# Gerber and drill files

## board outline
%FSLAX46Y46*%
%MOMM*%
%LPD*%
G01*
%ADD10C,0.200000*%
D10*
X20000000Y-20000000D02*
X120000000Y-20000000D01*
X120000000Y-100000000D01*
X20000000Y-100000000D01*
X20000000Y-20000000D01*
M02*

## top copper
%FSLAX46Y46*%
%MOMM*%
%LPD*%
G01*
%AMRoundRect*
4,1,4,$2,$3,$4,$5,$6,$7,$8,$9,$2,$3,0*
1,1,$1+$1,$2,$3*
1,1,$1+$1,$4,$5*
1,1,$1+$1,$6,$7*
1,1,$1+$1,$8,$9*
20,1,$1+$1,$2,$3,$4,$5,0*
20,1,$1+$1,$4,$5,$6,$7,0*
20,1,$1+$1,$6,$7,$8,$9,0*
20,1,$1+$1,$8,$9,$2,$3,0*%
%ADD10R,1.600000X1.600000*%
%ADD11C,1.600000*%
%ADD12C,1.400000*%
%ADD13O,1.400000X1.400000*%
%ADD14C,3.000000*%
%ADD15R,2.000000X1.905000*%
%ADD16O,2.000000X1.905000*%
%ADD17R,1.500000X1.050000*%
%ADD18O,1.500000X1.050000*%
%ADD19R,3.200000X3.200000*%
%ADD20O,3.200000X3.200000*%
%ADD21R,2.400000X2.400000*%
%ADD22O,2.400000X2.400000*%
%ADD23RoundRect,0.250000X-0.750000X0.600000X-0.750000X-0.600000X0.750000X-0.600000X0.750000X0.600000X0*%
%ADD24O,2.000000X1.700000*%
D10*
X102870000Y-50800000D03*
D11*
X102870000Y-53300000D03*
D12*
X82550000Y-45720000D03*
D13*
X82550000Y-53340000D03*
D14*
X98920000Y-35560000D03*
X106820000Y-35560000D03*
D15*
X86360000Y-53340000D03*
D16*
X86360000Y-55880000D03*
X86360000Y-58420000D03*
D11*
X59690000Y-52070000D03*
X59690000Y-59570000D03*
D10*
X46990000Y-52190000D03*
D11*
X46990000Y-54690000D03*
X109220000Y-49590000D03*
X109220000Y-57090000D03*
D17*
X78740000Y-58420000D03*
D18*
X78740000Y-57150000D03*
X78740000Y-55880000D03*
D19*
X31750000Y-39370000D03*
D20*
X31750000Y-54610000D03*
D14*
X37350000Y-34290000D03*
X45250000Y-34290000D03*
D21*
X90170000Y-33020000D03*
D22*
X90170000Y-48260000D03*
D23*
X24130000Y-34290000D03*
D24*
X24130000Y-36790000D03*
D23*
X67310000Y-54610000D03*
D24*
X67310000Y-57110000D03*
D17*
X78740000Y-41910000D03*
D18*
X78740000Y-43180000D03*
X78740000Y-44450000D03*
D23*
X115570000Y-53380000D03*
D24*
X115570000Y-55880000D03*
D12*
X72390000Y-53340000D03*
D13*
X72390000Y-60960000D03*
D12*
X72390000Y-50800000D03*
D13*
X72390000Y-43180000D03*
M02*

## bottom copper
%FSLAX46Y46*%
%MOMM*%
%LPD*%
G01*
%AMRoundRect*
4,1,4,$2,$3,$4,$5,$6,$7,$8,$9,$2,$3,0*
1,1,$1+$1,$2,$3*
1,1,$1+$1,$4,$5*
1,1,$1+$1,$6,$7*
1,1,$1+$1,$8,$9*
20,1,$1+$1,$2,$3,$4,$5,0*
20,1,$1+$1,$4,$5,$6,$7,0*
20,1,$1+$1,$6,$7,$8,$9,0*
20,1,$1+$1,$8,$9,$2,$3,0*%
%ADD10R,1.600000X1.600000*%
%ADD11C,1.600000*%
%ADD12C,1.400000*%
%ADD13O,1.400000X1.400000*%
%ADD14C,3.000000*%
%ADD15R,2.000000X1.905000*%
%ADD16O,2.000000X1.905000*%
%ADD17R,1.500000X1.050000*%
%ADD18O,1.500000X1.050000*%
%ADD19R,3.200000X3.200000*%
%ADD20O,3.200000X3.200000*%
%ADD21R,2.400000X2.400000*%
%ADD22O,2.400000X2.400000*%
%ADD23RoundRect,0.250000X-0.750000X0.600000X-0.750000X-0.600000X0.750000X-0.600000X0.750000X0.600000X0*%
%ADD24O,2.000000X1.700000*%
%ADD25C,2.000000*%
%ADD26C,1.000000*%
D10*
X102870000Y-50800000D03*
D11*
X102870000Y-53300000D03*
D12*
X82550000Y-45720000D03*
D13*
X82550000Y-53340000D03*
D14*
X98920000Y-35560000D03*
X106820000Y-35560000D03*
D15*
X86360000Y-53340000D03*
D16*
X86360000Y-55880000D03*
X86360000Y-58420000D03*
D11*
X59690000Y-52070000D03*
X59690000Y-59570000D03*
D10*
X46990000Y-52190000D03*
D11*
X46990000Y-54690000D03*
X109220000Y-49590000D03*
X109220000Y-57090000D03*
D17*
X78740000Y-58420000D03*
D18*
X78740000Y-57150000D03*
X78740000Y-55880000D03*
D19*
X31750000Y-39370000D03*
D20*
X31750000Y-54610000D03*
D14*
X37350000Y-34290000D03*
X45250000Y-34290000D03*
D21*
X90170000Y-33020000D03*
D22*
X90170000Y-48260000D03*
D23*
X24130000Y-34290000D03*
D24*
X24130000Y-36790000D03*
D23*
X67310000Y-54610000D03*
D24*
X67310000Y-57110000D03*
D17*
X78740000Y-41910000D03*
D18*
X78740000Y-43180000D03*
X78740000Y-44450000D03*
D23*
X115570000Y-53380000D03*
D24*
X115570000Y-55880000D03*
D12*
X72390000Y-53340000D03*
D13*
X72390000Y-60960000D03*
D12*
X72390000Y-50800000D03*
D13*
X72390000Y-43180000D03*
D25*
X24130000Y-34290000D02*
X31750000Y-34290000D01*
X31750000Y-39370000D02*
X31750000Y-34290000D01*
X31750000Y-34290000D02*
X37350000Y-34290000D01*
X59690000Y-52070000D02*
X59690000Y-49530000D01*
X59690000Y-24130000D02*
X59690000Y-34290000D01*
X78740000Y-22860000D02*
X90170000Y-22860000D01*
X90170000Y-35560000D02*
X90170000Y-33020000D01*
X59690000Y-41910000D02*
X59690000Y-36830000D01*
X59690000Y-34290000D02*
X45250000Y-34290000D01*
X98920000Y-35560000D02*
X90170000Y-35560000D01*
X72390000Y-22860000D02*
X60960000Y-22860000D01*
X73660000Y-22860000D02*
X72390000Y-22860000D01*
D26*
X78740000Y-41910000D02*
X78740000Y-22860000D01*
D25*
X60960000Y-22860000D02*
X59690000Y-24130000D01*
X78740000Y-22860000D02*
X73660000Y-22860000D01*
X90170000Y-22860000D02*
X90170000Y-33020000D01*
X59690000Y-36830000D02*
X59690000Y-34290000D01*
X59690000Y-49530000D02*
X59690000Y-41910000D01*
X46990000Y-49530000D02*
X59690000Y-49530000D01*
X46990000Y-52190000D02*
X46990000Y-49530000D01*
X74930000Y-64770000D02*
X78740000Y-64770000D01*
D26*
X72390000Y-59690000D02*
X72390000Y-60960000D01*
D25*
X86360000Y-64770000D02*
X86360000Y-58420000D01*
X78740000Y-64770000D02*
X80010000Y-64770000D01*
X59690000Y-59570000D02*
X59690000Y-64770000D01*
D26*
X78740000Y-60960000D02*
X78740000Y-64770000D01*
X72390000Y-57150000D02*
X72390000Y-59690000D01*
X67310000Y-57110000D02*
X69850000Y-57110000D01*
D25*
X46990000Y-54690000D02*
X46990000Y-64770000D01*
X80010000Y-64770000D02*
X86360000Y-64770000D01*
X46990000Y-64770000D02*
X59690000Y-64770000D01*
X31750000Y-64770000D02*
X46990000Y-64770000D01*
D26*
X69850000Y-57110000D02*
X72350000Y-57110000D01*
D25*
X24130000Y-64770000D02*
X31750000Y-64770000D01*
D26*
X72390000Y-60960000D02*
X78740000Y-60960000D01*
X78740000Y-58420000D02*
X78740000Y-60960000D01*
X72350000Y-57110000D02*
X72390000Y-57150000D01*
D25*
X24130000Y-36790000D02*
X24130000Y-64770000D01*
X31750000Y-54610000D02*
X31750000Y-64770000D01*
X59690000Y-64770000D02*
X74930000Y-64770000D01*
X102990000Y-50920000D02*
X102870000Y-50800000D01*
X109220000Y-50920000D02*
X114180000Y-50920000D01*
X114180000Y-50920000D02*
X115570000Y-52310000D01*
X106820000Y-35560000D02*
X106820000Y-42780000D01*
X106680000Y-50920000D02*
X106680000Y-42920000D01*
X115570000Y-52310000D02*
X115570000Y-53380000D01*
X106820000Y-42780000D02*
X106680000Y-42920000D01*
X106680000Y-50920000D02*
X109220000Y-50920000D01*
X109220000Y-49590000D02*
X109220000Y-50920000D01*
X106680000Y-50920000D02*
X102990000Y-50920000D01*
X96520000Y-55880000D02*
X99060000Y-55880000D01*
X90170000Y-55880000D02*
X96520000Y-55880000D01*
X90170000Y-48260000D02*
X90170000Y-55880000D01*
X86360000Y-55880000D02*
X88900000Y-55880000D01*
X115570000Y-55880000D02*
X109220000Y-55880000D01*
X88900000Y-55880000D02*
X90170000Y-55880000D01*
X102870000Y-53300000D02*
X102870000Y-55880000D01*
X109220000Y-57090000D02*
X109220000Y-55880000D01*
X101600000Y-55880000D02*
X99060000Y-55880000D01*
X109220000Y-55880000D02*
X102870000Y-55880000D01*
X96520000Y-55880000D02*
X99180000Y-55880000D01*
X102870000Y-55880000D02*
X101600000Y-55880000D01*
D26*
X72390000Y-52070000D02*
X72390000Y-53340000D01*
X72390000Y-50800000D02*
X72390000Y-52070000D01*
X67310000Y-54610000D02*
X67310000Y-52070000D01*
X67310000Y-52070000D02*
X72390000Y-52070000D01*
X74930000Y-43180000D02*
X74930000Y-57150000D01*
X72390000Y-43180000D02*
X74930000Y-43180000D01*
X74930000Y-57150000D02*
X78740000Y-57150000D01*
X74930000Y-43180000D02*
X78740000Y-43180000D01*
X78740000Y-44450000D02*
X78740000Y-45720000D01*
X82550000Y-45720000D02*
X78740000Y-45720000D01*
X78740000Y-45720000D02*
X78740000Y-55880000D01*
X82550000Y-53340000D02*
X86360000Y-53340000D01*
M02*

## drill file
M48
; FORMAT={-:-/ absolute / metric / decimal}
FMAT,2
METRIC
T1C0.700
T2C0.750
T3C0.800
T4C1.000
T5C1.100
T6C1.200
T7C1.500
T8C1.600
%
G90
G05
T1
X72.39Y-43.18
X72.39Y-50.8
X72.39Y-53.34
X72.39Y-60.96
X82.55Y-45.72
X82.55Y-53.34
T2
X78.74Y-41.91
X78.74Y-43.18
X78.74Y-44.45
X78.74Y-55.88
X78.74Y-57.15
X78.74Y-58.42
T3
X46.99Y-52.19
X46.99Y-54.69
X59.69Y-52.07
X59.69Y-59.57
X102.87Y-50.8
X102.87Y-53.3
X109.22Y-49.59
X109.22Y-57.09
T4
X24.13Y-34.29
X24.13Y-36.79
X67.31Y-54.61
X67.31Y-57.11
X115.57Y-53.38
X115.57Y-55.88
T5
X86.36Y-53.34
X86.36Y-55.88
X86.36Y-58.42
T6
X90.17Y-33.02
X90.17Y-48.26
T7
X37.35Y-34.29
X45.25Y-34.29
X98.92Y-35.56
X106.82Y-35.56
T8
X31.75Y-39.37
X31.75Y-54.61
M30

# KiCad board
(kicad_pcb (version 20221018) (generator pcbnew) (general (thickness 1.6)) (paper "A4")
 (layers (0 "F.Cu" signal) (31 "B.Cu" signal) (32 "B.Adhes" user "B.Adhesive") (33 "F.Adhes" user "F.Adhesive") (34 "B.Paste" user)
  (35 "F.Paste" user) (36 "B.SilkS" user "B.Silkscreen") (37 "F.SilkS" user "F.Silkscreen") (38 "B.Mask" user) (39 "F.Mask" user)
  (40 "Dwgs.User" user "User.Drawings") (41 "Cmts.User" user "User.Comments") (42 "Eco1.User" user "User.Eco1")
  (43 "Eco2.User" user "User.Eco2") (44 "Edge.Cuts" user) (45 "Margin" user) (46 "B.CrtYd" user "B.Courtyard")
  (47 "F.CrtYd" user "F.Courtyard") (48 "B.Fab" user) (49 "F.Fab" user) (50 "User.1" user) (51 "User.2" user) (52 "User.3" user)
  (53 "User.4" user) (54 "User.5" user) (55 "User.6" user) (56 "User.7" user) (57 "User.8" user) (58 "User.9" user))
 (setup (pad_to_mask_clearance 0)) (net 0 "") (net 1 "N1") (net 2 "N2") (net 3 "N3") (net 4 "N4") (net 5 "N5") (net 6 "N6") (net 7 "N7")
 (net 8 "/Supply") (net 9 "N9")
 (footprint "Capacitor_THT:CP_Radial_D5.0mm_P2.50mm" (layer "F.Cu") (at 102.87 50.8 -90)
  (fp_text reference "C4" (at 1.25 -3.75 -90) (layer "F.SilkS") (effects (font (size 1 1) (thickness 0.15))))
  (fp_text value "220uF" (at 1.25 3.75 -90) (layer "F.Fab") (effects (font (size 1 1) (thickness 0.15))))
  (pad "1" thru_hole rect (at 0 0 270) (size 1.6 1.6) (drill 0.8) (layers "*.Cu" "*.Mask") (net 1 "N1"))
  (pad "2" thru_hole circle (at 2.5 0 270) (size 1.6 1.6) (drill 0.8) (layers "*.Cu" "*.Mask") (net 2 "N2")))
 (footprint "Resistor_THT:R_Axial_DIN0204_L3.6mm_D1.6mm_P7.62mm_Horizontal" (layer "F.Cu") (at 82.55 45.72 -90)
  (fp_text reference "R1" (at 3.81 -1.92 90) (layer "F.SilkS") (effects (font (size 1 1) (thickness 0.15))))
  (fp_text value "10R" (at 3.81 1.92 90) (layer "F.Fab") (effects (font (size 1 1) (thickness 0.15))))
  (pad "1" thru_hole circle (at 0 0 270) (size 1.4 1.4) (drill 0.7) (layers "*.Cu" "*.Mask") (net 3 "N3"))
  (pad "2" thru_hole oval (at 7.62 0 270) (size 1.4 1.4) (drill 0.7) (layers "*.Cu" "*.Mask") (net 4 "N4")))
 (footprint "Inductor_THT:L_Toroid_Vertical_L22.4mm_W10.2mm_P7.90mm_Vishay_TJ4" (layer "F.Cu") (at 98.92 35.56 90)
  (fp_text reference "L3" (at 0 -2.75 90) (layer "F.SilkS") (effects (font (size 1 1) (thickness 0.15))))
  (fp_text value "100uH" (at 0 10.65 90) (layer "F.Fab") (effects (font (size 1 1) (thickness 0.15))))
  (pad "1" thru_hole circle (at 0 0 90) (size 3 3) (drill 1.5) (layers "*.Cu" "*.Mask") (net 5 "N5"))
  (pad "2" thru_hole circle (at 0 7.9 90) (size 3 3) (drill 1.5) (layers "*.Cu" "*.Mask") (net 1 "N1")))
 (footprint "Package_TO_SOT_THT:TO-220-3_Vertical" (layer "F.Cu") (at 86.36 53.34 -90)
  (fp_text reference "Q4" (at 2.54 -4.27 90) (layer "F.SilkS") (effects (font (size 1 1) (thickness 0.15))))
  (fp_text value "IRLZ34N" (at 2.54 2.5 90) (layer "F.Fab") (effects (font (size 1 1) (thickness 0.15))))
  (pad "1" thru_hole rect (at 0 0 270) (size 1.905 2) (drill 1.1) (layers "*.Cu" "*.Mask") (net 4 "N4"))
  (pad "2" thru_hole oval (at 2.54 0 270) (size 1.905 2) (drill 1.1) (layers "*.Cu" "*.Mask") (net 2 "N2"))
  (pad "3" thru_hole oval (at 5.08 0 270) (size 1.905 2) (drill 1.1) (layers "*.Cu" "*.Mask") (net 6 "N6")))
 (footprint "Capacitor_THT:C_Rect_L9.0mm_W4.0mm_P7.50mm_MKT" (layer "F.Cu") (at 59.69 52.07 -90)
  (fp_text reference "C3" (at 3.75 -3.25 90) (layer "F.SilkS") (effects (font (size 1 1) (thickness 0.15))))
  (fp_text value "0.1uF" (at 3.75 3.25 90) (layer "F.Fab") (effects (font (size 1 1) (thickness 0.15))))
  (pad "1" thru_hole circle (at 0 0 270) (size 1.6 1.6) (drill 0.8) (layers "*.Cu" "*.Mask") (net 5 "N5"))
  (pad "2" thru_hole circle (at 7.5 0 270) (size 1.6 1.6) (drill 0.8) (layers "*.Cu" "*.Mask") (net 6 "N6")))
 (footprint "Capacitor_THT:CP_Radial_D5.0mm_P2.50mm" (layer "F.Cu") (at 46.99 52.19 -90)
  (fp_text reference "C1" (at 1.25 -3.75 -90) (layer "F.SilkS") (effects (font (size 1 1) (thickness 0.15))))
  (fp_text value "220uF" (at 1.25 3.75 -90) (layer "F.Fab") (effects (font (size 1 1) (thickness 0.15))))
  (pad "1" thru_hole rect (at 0 0 270) (size 1.6 1.6) (drill 0.8) (layers "*.Cu" "*.Mask") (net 5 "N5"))
  (pad "2" thru_hole circle (at 2.5 0 270) (size 1.6 1.6) (drill 0.8) (layers "*.Cu" "*.Mask") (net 6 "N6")))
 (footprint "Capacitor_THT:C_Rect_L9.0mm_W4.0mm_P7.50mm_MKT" (layer "F.Cu") (at 109.22 49.59 -90)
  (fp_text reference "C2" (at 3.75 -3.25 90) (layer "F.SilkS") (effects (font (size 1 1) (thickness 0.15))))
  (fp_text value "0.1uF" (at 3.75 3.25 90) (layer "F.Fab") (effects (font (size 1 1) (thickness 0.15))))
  (pad "1" thru_hole circle (at 0 0 270) (size 1.6 1.6) (drill 0.8) (layers "*.Cu" "*.Mask") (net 1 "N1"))
  (pad "2" thru_hole circle (at 7.5 0 270) (size 1.6 1.6) (drill 0.8) (layers "*.Cu" "*.Mask") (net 2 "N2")))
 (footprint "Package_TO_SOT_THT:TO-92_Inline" (layer "F.Cu") (at 78.74 58.42 90)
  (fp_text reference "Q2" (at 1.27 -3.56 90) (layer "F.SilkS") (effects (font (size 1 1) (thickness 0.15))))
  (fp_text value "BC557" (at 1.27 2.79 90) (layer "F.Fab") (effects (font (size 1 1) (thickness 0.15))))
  (pad "1" thru_hole rect (at 0 0 90) (size 1.05 1.5) (drill 0.75) (layers "*.Cu" "*.Mask") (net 6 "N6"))
  (pad "2" thru_hole oval (at 1.27 0 90) (size 1.05 1.5) (drill 0.75) (layers "*.Cu" "*.Mask") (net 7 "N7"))
  (pad "3" thru_hole oval (at 2.54 0 90) (size 1.05 1.5) (drill 0.75) (layers "*.Cu" "*.Mask") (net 3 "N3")))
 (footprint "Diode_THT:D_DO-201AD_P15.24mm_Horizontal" (layer "F.Cu") (at 31.75 39.37 -90)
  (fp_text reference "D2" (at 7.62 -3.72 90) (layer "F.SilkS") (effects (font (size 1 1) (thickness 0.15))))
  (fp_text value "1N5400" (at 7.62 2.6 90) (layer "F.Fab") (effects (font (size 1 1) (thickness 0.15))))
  (pad "1" thru_hole rect (at 0 0 270) (size 3.2 3.2) (drill 1.6) (layers "*.Cu" "*.Mask") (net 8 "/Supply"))
  (pad "2" thru_hole oval (at 15.24 0 270) (size 3.2 3.2) (drill 1.6) (layers "*.Cu" "*.Mask") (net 6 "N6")))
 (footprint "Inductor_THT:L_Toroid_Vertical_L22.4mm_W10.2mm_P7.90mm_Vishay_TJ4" (layer "F.Cu") (at 37.35 34.29 90)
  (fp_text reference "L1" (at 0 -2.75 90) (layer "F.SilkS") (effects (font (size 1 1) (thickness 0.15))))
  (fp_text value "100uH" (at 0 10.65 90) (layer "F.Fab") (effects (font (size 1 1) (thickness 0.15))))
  (pad "1" thru_hole circle (at 0 0 90) (size 3 3) (drill 1.5) (layers "*.Cu" "*.Mask") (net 8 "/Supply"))
  (pad "2" thru_hole circle (at 0 7.9 90) (size 3 3) (drill 1.5) (layers "*.Cu" "*.Mask") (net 5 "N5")))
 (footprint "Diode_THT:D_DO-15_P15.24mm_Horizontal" (layer "F.Cu") (at 90.17 33.02 -90)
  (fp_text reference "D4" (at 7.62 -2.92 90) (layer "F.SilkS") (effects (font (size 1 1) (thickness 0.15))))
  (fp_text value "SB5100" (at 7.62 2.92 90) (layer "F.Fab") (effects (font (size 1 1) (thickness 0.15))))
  (pad "1" thru_hole rect (at 0 0 270) (size 2.4 2.4) (drill 1.2) (layers "*.Cu" "*.Mask") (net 5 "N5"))
  (pad "2" thru_hole oval (at 15.24 0 270) (size 2.4 2.4) (drill 1.2) (layers "*.Cu" "*.Mask") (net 2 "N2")))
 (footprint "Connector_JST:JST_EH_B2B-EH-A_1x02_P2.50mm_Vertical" (layer "F.Cu") (at 24.13 34.29 -90)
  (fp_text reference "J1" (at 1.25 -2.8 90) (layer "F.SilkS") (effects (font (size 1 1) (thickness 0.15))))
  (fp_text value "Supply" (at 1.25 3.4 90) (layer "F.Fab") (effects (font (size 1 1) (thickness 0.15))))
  (pad "1" thru_hole roundrect (at 0 0 270) (size 1.7 2) (drill 1) (layers "*.Cu" "*.Mask") (roundrect_rratio 0.147059) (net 8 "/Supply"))
  (pad "2" thru_hole oval (at 2.5 0 270) (size 1.7 2) (drill 1) (layers "*.Cu" "*.Mask") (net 6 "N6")))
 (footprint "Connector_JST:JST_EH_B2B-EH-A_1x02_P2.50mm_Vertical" (layer "F.Cu") (at 67.31 54.61 -90)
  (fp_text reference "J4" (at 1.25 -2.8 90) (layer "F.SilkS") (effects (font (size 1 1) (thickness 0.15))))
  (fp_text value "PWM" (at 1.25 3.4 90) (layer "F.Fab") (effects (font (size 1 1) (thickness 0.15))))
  (pad "1" thru_hole roundrect (at 0 0 270) (size 1.7 2) (drill 1) (layers "*.Cu" "*.Mask") (roundrect_rratio 0.147059) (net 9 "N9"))
  (pad "2" thru_hole oval (at 2.5 0 270) (size 1.7 2) (drill 1) (layers "*.Cu" "*.Mask") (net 6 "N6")))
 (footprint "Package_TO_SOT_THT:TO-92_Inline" (layer "F.Cu") (at 78.74 41.91 -90)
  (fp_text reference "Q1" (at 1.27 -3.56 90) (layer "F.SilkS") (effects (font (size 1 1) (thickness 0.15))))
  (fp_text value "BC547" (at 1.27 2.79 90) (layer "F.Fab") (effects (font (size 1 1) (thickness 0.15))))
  (pad "1" thru_hole rect (at 0 0 270) (size 1.05 1.5) (drill 0.75) (layers "*.Cu" "*.Mask") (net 5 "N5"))
  (pad "2" thru_hole oval (at 1.27 0 270) (size 1.05 1.5) (drill 0.75) (layers "*.Cu" "*.Mask") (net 7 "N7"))
  (pad "3" thru_hole oval (at 2.54 0 270) (size 1.05 1.5) (drill 0.75) (layers "*.Cu" "*.Mask") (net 3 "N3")))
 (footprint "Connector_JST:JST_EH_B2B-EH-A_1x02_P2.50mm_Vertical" (layer "F.Cu") (at 115.57 53.38 -90)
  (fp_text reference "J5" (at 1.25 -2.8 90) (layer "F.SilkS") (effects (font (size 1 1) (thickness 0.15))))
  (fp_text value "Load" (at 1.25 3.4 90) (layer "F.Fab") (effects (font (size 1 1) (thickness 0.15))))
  (pad "1" thru_hole roundrect (at 0 0 270) (size 1.7 2) (drill 1) (layers "*.Cu" "*.Mask") (roundrect_rratio 0.147059) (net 1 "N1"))
  (pad "2" thru_hole oval (at 2.5 0 270) (size 1.7 2) (drill 1) (layers "*.Cu" "*.Mask") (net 2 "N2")))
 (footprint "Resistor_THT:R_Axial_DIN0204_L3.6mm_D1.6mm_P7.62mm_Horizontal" (layer "F.Cu") (at 72.39 53.34 -90)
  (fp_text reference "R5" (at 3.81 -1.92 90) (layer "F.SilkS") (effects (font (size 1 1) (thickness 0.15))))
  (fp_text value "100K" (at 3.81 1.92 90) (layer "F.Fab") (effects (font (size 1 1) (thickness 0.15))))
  (pad "1" thru_hole circle (at 0 0 270) (size 1.4 1.4) (drill 0.7) (layers "*.Cu" "*.Mask") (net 9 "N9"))
  (pad "2" thru_hole oval (at 7.62 0 270) (size 1.4 1.4) (drill 0.7) (layers "*.Cu" "*.Mask") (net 6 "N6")))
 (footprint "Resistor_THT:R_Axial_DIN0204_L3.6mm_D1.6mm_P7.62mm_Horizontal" (layer "F.Cu") (at 72.39 50.8 90)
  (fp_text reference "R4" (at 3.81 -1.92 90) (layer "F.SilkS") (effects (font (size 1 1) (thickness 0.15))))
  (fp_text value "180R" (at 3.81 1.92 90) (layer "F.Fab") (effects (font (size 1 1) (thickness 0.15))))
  (pad "1" thru_hole circle (at 0 0 90) (size 1.4 1.4) (drill 0.7) (layers "*.Cu" "*.Mask") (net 9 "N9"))
  (pad "2" thru_hole oval (at 7.62 0 90) (size 1.4 1.4) (drill 0.7) (layers "*.Cu" "*.Mask") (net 7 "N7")))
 (gr_rect (start 20 20) (end 120 100) (stroke (width 0.2) (type default)) (fill none) (layer "Edge.Cuts"))
 (segment (start 24.13 34.29) (end 31.75 34.29) (width 2) (layer "B.Cu") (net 8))
 (segment (start 31.75 39.37) (end 31.75 34.29) (width 2) (layer "B.Cu") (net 8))
 (segment (start 31.75 34.29) (end 37.35 34.29) (width 2) (layer "B.Cu") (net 8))
 (segment (start 59.69 52.07) (end 59.69 49.53) (width 2) (layer "B.Cu") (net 5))
 (segment (start 59.69 24.13) (end 59.69 34.29) (width 2) (layer "B.Cu") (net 5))
 (segment (start 78.74 22.86) (end 90.17 22.86) (width 2) (layer "B.Cu") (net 5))
 (segment (start 90.17 35.56) (end 90.17 33.02) (width 2) (layer "B.Cu") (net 5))
 (segment (start 59.69 41.91) (end 59.69 36.83) (width 2) (layer "B.Cu") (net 5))
 (segment (start 59.69 34.29) (end 45.25 34.29) (width 2) (layer "B.Cu") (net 5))
 (segment (start 98.92 35.56) (end 90.17 35.56) (width 2) (layer "B.Cu") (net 5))
 (segment (start 72.39 22.86) (end 60.96 22.86) (width 2) (layer "B.Cu") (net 5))
 (segment (start 73.66 22.86) (end 72.39 22.86) (width 2) (layer "B.Cu") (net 5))
 (segment (start 78.74 41.91) (end 78.74 22.86) (width 1) (layer "B.Cu") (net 5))
 (segment (start 60.96 22.86) (end 59.69 24.13) (width 2) (layer "B.Cu") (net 5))
 (segment (start 78.74 22.86) (end 73.66 22.86) (width 2) (layer "B.Cu") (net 5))
 (segment (start 90.17 22.86) (end 90.17 33.02) (width 2) (layer "B.Cu") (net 5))
 (segment (start 59.69 36.83) (end 59.69 34.29) (width 2) (layer "B.Cu") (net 5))
 (segment (start 59.69 49.53) (end 59.69 41.91) (width 2) (layer "B.Cu") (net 5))
 (segment (start 46.99 49.53) (end 59.69 49.53) (width 2) (layer "B.Cu") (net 5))
 (segment (start 46.99 52.19) (end 46.99 49.53) (width 2) (layer "B.Cu") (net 5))
 (segment (start 74.93 64.77) (end 78.74 64.77) (width 2) (layer "B.Cu") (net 6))
 (segment (start 72.39 59.69) (end 72.39 60.96) (width 1) (layer "B.Cu") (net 6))
 (segment (start 86.36 64.77) (end 86.36 58.42) (width 2) (layer "B.Cu") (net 6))
 (segment (start 78.74 64.77) (end 80.01 64.77) (width 2) (layer "B.Cu") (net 6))
 (segment (start 59.69 59.57) (end 59.69 64.77) (width 2) (layer "B.Cu") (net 6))
 (segment (start 78.74 60.96) (end 78.74 64.77) (width 1) (layer "B.Cu") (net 6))
 (segment (start 72.39 57.15) (end 72.39 59.69) (width 1) (layer "B.Cu") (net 6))
 (segment (start 67.31 57.11) (end 69.85 57.11) (width 1) (layer "B.Cu") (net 6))
 (segment (start 46.99 54.69) (end 46.99 64.77) (width 2) (layer "B.Cu") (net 6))
 (segment (start 80.01 64.77) (end 86.36 64.77) (width 2) (layer "B.Cu") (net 6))
 (segment (start 46.99 64.77) (end 59.69 64.77) (width 2) (layer "B.Cu") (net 6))
 (segment (start 31.75 64.77) (end 46.99 64.77) (width 2) (layer "B.Cu") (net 6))
 (segment (start 69.85 57.11) (end 72.35 57.11) (width 1) (layer "B.Cu") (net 6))
 (segment (start 24.13 64.77) (end 31.75 64.77) (width 2) (layer "B.Cu") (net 6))
 (segment (start 72.39 60.96) (end 78.74 60.96) (width 1) (layer "B.Cu") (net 6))
 (segment (start 78.74 58.42) (end 78.74 60.96) (width 1) (layer "B.Cu") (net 6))
 (segment (start 72.35 57.11) (end 72.39 57.15) (width 1) (layer "B.Cu") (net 6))
 (segment (start 24.13 36.79) (end 24.13 64.77) (width 2) (layer "B.Cu") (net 6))
 (segment (start 31.75 54.61) (end 31.75 64.77) (width 2) (layer "B.Cu") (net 6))
 (segment (start 59.69 64.77) (end 74.93 64.77) (width 2) (layer "B.Cu") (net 6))
 (segment (start 102.99 50.92) (end 102.87 50.8) (width 2) (layer "B.Cu") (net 1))
 (segment (start 109.22 50.92) (end 114.18 50.92) (width 2) (layer "B.Cu") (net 1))
 (segment (start 114.18 50.92) (end 115.57 52.31) (width 2) (layer "B.Cu") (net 1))
 (segment (start 106.82 35.56) (end 106.82 42.78) (width 2) (layer "B.Cu") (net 1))
 (segment (start 106.68 50.92) (end 106.68 42.92) (width 2) (layer "B.Cu") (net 1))
 (segment (start 115.57 52.31) (end 115.57 53.38) (width 2) (layer "B.Cu") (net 1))
 (segment (start 106.82 42.78) (end 106.68 42.92) (width 2) (layer "B.Cu") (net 1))
 (segment (start 106.68 50.92) (end 109.22 50.92) (width 2) (layer "B.Cu") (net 1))
 (segment (start 109.22 49.59) (end 109.22 50.92) (width 2) (layer "B.Cu") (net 1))
 (segment (start 106.68 50.92) (end 102.99 50.92) (width 2) (layer "B.Cu") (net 1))
 (segment (start 96.52 55.88) (end 99.06 55.88) (width 2) (layer "B.Cu") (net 2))
 (segment (start 90.17 55.88) (end 96.52 55.88) (width 2) (layer "B.Cu") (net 2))
 (segment (start 90.17 48.26) (end 90.17 55.88) (width 2) (layer "B.Cu") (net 2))
 (segment (start 86.36 55.88) (end 88.9 55.88) (width 2) (layer "B.Cu") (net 2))
 (segment (start 115.57 55.88) (end 109.22 55.88) (width 2) (layer "B.Cu") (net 2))
 (segment (start 88.9 55.88) (end 90.17 55.88) (width 2) (layer "B.Cu") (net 2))
 (segment (start 102.87 53.3) (end 102.87 55.88) (width 2) (layer "B.Cu") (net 2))
 (segment (start 109.22 57.09) (end 109.22 55.88) (width 2) (layer "B.Cu") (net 2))
 (segment (start 101.6 55.88) (end 99.06 55.88) (width 2) (layer "B.Cu") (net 2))
 (segment (start 109.22 55.88) (end 102.87 55.88) (width 2) (layer "B.Cu") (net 2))
 (segment (start 96.52 55.88) (end 99.18 55.88) (width 2) (layer "B.Cu") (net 2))
 (segment (start 102.87 55.88) (end 101.6 55.88) (width 2) (layer "B.Cu") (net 2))
 (segment (start 72.39 52.07) (end 72.39 53.34) (width 1) (layer "B.Cu") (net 9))
 (segment (start 72.39 50.8) (end 72.39 52.07) (width 1) (layer "B.Cu") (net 9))
 (segment (start 67.31 54.61) (end 67.31 52.07) (width 1) (layer "B.Cu") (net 9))
 (segment (start 67.31 52.07) (end 72.39 52.07) (width 1) (layer "B.Cu") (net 9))
 (segment (start 74.93 43.18) (end 74.93 57.15) (width 1) (layer "B.Cu") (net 7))
 (segment (start 72.39 43.18) (end 74.93 43.18) (width 1) (layer "B.Cu") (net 7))
 (segment (start 74.93 57.15) (end 78.74 57.15) (width 1) (layer "B.Cu") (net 7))
 (segment (start 74.93 43.18) (end 78.74 43.18) (width 1) (layer "B.Cu") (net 7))
 (segment (start 78.74 44.45) (end 78.74 45.72) (width 1) (layer "B.Cu") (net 3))
 (segment (start 82.55 45.72) (end 78.74 45.72) (width 1) (layer "B.Cu") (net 3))
 (segment (start 78.74 45.72) (end 78.74 55.88) (width 1) (layer "B.Cu") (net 3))
 (segment (start 82.55 53.34) (end 86.36 53.34) (width 1) (layer "B.Cu") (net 4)))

